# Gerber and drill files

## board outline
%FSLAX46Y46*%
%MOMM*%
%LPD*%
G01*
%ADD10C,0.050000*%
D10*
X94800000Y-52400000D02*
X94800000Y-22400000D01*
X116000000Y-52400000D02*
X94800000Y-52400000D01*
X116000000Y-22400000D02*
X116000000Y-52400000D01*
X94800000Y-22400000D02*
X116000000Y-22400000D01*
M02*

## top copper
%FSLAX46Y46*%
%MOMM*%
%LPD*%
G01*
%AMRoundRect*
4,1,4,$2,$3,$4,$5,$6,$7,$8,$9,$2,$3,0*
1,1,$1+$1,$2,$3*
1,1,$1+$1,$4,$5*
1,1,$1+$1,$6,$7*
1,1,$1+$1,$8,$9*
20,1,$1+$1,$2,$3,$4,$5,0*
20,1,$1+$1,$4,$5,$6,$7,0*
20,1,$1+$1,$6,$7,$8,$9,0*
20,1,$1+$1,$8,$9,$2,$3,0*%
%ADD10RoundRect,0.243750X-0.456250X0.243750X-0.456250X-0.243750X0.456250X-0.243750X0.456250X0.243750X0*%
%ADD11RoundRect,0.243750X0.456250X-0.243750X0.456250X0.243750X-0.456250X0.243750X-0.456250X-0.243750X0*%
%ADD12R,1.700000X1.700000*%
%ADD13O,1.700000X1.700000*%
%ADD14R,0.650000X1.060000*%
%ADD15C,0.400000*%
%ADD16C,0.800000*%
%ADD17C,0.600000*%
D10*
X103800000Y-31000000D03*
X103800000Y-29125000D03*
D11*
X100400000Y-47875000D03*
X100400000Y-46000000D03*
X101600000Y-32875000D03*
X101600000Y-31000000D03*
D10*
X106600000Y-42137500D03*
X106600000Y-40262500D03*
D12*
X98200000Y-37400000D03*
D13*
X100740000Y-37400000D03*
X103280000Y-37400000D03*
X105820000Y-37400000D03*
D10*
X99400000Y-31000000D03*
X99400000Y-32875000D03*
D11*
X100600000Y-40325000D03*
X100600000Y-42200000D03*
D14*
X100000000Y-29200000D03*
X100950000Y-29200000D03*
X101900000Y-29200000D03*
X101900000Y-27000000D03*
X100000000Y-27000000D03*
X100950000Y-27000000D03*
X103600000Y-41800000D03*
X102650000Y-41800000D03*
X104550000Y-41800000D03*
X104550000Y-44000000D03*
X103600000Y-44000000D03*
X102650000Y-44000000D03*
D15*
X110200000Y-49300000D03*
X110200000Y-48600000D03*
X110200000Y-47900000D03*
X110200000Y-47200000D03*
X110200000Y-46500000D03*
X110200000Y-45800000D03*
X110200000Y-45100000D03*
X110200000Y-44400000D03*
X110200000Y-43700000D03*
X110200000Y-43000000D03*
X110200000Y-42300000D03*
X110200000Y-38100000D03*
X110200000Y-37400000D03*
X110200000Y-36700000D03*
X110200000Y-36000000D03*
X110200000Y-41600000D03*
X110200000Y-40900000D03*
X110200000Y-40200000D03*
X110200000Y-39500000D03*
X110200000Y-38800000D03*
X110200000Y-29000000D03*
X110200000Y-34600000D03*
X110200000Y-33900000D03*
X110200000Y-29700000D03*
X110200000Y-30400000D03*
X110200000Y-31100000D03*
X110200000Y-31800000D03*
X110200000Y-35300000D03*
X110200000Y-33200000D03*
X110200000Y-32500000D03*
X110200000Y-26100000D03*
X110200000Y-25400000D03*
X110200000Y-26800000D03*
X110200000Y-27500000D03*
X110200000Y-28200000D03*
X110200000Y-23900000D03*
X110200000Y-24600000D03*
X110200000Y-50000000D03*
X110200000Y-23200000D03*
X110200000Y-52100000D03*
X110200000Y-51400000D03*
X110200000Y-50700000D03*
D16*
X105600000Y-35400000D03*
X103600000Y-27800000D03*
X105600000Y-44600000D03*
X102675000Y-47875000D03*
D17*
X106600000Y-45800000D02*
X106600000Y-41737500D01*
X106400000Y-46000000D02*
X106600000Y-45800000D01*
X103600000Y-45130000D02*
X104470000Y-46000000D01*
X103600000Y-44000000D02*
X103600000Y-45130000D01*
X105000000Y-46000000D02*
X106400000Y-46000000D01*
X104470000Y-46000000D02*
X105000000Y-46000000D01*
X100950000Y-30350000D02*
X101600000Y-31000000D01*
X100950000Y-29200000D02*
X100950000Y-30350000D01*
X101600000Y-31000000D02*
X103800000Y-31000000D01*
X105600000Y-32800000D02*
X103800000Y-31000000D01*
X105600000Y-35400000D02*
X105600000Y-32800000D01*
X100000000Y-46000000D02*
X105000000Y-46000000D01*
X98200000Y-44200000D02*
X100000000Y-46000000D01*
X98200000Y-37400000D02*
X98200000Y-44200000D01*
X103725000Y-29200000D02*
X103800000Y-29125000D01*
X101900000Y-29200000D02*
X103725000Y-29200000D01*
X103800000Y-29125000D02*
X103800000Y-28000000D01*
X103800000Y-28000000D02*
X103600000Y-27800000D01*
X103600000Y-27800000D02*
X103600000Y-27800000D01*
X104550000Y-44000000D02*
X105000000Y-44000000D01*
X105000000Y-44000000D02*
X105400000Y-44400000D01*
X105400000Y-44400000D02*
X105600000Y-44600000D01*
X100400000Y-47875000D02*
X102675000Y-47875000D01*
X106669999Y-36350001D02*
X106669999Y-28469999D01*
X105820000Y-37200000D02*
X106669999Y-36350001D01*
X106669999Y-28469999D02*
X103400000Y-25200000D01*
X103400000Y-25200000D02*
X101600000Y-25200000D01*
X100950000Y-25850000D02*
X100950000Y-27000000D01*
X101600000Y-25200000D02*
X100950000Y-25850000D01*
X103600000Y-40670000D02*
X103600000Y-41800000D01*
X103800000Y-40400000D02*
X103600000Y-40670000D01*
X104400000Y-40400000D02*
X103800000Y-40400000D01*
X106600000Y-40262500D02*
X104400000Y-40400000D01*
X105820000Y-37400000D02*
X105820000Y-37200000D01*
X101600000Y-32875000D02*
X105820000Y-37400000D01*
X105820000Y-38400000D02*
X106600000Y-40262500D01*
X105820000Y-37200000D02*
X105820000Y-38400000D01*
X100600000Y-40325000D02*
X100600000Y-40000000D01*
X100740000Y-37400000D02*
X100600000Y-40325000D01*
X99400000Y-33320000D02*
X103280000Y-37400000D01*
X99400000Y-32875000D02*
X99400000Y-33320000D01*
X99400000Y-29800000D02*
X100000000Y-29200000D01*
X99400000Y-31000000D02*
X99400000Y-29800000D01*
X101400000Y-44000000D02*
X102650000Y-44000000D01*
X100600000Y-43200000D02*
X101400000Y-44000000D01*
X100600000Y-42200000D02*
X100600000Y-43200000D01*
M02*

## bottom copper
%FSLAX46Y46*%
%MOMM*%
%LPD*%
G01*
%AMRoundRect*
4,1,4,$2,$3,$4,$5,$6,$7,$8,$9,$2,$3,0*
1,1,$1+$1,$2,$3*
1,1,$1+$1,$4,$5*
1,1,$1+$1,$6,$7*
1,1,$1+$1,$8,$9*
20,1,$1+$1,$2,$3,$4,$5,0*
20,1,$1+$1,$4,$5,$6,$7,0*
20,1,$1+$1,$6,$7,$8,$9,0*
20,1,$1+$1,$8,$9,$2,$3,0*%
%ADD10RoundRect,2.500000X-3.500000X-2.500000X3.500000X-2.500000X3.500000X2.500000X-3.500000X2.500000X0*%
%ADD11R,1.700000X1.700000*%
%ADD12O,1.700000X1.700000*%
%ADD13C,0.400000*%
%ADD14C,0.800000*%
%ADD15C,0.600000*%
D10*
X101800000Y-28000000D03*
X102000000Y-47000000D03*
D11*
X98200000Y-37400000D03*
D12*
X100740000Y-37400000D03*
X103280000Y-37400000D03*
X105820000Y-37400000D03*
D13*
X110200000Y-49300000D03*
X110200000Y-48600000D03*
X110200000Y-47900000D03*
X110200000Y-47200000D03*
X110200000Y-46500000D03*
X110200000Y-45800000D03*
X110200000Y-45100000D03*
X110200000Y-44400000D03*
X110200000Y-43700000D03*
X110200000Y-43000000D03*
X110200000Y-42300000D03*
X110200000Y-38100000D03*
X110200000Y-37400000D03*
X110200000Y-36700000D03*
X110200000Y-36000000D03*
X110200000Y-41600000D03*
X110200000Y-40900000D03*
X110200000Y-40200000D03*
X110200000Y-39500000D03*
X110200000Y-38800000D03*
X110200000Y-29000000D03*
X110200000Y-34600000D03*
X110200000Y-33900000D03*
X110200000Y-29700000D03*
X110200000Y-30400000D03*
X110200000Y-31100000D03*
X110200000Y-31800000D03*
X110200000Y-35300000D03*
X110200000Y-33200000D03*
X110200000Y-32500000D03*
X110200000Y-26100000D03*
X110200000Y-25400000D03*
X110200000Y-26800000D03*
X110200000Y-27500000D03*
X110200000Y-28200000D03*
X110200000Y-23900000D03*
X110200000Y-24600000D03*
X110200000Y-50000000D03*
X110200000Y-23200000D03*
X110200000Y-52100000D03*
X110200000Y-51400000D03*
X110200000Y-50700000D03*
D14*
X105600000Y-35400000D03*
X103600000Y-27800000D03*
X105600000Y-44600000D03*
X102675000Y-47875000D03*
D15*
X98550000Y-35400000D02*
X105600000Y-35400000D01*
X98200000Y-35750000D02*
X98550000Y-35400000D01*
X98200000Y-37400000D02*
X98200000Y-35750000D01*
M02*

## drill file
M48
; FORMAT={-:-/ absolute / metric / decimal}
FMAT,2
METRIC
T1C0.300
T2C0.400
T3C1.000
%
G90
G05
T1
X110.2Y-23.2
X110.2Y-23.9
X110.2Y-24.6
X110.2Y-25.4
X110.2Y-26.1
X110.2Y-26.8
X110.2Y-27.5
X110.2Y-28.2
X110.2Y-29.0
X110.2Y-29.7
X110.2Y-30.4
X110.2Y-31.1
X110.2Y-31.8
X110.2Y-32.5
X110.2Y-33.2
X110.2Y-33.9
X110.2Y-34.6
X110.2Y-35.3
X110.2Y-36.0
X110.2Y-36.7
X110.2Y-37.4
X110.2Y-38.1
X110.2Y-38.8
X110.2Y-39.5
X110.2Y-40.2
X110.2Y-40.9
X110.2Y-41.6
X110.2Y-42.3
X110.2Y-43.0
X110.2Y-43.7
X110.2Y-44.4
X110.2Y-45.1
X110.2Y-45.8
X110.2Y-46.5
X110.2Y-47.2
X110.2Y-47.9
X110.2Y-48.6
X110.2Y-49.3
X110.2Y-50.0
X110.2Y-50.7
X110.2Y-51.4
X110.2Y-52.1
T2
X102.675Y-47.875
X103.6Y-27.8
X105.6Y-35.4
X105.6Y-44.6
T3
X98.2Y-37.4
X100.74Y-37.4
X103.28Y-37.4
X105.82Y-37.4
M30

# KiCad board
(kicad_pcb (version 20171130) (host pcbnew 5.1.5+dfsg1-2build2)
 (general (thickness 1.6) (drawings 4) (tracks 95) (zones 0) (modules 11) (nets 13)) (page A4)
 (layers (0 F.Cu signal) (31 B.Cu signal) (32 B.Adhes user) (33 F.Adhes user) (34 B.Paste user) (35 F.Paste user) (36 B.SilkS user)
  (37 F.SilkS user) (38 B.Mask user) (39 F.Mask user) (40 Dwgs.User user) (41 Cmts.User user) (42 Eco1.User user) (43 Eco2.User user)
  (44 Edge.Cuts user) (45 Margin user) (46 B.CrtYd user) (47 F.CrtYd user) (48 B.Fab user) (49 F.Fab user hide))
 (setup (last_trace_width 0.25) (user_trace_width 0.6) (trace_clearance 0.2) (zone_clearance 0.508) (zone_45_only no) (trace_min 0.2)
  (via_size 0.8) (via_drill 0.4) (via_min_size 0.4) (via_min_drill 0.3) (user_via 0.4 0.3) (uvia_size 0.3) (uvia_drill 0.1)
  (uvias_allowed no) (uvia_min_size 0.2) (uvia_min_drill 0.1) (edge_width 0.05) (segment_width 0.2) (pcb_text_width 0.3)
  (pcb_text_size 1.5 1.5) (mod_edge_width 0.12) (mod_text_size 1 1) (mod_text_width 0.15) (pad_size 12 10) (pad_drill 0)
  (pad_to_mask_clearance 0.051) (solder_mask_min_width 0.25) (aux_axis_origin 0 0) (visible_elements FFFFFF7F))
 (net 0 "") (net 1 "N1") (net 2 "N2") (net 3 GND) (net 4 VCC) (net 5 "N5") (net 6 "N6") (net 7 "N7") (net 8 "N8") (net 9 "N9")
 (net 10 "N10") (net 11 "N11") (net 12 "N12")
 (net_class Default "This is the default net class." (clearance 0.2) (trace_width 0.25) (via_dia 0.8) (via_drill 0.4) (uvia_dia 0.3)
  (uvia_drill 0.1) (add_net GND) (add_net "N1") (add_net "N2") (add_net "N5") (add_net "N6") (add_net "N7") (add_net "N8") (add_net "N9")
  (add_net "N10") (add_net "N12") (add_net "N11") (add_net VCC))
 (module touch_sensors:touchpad (layer B.Cu) (at 101.8 28)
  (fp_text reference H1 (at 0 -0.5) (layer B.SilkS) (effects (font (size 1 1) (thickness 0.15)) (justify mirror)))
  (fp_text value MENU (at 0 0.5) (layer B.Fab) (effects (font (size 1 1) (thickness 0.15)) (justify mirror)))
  (pad 1 smd roundrect (at 0 0) (size 12 10) (layers B.Cu) (roundrect_rratio 0.25) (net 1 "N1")))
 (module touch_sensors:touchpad (layer B.Cu) (at 101.85 47)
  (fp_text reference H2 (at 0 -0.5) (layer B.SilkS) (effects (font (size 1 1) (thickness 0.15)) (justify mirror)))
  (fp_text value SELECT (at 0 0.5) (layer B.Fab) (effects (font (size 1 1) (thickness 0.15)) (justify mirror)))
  (pad 1 smd roundrect (at 0.15 0) (size 12 10) (layers B.Cu) (roundrect_rratio 0.25) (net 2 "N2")))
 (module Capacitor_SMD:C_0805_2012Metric (layer F.Cu) (at 103.8 30.0625 270)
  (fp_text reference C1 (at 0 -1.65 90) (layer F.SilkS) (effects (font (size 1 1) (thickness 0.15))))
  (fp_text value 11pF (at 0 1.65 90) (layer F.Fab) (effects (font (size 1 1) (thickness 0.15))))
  (pad 2 smd roundrect (at 0.9375 0 270) (size 0.975 1.4) (layers F.Cu F.Paste F.Mask) (roundrect_rratio 0.25) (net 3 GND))
  (pad 1 smd roundrect (at -0.9375 0 270) (size 0.975 1.4) (layers F.Cu F.Paste F.Mask) (roundrect_rratio 0.25) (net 1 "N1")))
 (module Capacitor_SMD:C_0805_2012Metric (layer F.Cu) (at 100.4 46.9375 90)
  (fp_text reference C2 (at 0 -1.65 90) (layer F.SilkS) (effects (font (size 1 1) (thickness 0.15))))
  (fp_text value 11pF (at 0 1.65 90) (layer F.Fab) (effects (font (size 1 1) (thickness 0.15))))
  (pad 1 smd roundrect (at -0.9375 0 90) (size 0.975 1.4) (layers F.Cu F.Paste F.Mask) (roundrect_rratio 0.25) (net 2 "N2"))
  (pad 2 smd roundrect (at 0.9375 0 90) (size 0.975 1.4) (layers F.Cu F.Paste F.Mask) (roundrect_rratio 0.25) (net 3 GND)))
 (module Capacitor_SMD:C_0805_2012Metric (layer F.Cu) (at 101.6 31.9375 90)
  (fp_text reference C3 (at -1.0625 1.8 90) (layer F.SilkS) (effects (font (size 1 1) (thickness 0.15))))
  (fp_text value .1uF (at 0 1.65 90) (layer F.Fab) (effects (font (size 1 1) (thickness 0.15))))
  (pad 1 smd roundrect (at -0.9375 0 90) (size 0.975 1.4) (layers F.Cu F.Paste F.Mask) (roundrect_rratio 0.25) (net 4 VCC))
  (pad 2 smd roundrect (at 0.9375 0 90) (size 0.975 1.4) (layers F.Cu F.Paste F.Mask) (roundrect_rratio 0.25) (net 3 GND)))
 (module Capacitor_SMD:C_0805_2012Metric (layer F.Cu) (at 106.6 41.2 270)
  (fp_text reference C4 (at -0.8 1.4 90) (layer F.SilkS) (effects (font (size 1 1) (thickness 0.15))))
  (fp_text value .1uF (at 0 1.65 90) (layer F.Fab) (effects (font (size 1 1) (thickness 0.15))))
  (pad 2 smd roundrect (at 0.9375 0 270) (size 0.975 1.4) (layers F.Cu F.Paste F.Mask) (roundrect_rratio 0.25) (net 3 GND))
  (pad 1 smd roundrect (at -0.9375 0 270) (size 0.975 1.4) (layers F.Cu F.Paste F.Mask) (roundrect_rratio 0.25) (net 4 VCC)))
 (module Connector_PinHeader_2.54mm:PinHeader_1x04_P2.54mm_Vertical (layer F.Cu) (at 98.2 37.4 90)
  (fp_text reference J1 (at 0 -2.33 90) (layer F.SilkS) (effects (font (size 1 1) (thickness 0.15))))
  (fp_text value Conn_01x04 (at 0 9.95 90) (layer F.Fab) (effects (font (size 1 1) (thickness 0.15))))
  (pad 1 thru_hole rect (at 0 0 90) (size 1.7 1.7) (drill 1) (layers *.Cu *.Mask) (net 3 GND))
  (pad 2 thru_hole oval (at 0 2.54 90) (size 1.7 1.7) (drill 1) (layers *.Cu *.Mask) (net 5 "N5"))
  (pad 3 thru_hole oval (at 0 5.08 90) (size 1.7 1.7) (drill 1) (layers *.Cu *.Mask) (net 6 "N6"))
  (pad 4 thru_hole oval (at 0 7.62 90) (size 1.7 1.7) (drill 1) (layers *.Cu *.Mask) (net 4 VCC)))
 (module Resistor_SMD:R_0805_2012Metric (layer F.Cu) (at 99.4 31.9375 270)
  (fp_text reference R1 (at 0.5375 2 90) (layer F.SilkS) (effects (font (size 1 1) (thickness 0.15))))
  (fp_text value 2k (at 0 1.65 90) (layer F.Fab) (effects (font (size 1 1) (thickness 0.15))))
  (pad 1 smd roundrect (at -0.9375 0 270) (size 0.975 1.4) (layers F.Cu F.Paste F.Mask) (roundrect_rratio 0.25) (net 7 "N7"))
  (pad 2 smd roundrect (at 0.9375 0 270) (size 0.975 1.4) (layers F.Cu F.Paste F.Mask) (roundrect_rratio 0.25) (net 6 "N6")))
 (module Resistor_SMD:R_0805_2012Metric (layer F.Cu) (at 100.6 41.2625 90)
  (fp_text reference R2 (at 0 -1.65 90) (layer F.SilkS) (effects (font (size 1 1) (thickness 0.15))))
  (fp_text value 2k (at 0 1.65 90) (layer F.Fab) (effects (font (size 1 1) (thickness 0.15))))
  (pad 2 smd roundrect (at 0.9375 0 90) (size 0.975 1.4) (layers F.Cu F.Paste F.Mask) (roundrect_rratio 0.25) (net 5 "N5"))
  (pad 1 smd roundrect (at -0.9375 0 90) (size 0.975 1.4) (layers F.Cu F.Paste F.Mask) (roundrect_rratio 0.25) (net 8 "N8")))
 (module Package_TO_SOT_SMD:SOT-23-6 (layer F.Cu) (at 100.95 28.1 90)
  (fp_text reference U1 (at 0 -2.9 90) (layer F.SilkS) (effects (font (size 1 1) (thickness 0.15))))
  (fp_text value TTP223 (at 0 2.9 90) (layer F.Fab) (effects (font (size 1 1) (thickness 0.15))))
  (pad 1 smd rect (at -1.1 -0.95 90) (size 1.06 0.65) (layers F.Cu F.Paste F.Mask) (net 7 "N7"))
  (pad 2 smd rect (at -1.1 0 90) (size 1.06 0.65) (layers F.Cu F.Paste F.Mask) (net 3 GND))
  (pad 3 smd rect (at -1.1 0.95 90) (size 1.06 0.65) (layers F.Cu F.Paste F.Mask) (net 1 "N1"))
  (pad 4 smd rect (at 1.1 0.95 90) (size 1.06 0.65) (layers F.Cu F.Paste F.Mask) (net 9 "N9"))
  (pad 6 smd rect (at 1.1 -0.95 90) (size 1.06 0.65) (layers F.Cu F.Paste F.Mask) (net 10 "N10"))
  (pad 5 smd rect (at 1.1 0 90) (size 1.06 0.65) (layers F.Cu F.Paste F.Mask) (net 4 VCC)))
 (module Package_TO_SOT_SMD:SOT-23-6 (layer F.Cu) (at 103.6 42.9 90)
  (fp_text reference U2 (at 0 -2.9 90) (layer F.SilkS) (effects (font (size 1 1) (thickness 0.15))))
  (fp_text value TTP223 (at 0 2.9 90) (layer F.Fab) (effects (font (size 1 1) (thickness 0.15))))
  (pad 5 smd rect (at 1.1 0 90) (size 1.06 0.65) (layers F.Cu F.Paste F.Mask) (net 4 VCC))
  (pad 6 smd rect (at 1.1 -0.95 90) (size 1.06 0.65) (layers F.Cu F.Paste F.Mask) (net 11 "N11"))
  (pad 4 smd rect (at 1.1 0.95 90) (size 1.06 0.65) (layers F.Cu F.Paste F.Mask) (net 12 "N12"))
  (pad 3 smd rect (at -1.1 0.95 90) (size 1.06 0.65) (layers F.Cu F.Paste F.Mask) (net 2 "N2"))
  (pad 2 smd rect (at -1.1 0 90) (size 1.06 0.65) (layers F.Cu F.Paste F.Mask) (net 3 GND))
  (pad 1 smd rect (at -1.1 -0.95 90) (size 1.06 0.65) (layers F.Cu F.Paste F.Mask) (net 8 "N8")))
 (gr_line (start 94.8 52.4) (end 94.8 22.4) (layer Edge.Cuts) (width 0.05))
 (gr_line (start 116 52.4) (end 94.8 52.4) (layer Edge.Cuts) (width 0.05))
 (gr_line (start 116 22.4) (end 116 52.4) (layer Edge.Cuts) (width 0.05))
 (gr_line (start 94.8 22.4) (end 116 22.4) (layer Edge.Cuts) (width 0.05))
 (via (at 110.2 49.3) (size 0.4) (drill 0.3) (layers F.Cu B.Cu) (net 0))
 (via (at 110.2 48.6) (size 0.4) (drill 0.3) (layers F.Cu B.Cu) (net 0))
 (via (at 110.2 47.9) (size 0.4) (drill 0.3) (layers F.Cu B.Cu) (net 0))
 (via (at 110.2 47.2) (size 0.4) (drill 0.3) (layers F.Cu B.Cu) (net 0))
 (via (at 110.2 46.5) (size 0.4) (drill 0.3) (layers F.Cu B.Cu) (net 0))
 (via (at 110.2 45.8) (size 0.4) (drill 0.3) (layers F.Cu B.Cu) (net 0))
 (via (at 110.2 45.1) (size 0.4) (drill 0.3) (layers F.Cu B.Cu) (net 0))
 (via (at 110.2 44.4) (size 0.4) (drill 0.3) (layers F.Cu B.Cu) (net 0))
 (via (at 110.2 43.7) (size 0.4) (drill 0.3) (layers F.Cu B.Cu) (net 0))
 (via (at 110.2 43) (size 0.4) (drill 0.3) (layers F.Cu B.Cu) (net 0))
 (via (at 110.2 42.3) (size 0.4) (drill 0.3) (layers F.Cu B.Cu) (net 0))
 (via (at 110.2 38.1) (size 0.4) (drill 0.3) (layers F.Cu B.Cu) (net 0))
 (via (at 110.2 37.4) (size 0.4) (drill 0.3) (layers F.Cu B.Cu) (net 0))
 (via (at 110.2 36.7) (size 0.4) (drill 0.3) (layers F.Cu B.Cu) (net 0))
 (via (at 110.2 36) (size 0.4) (drill 0.3) (layers F.Cu B.Cu) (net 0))
 (via (at 110.2 41.6) (size 0.4) (drill 0.3) (layers F.Cu B.Cu) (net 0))
 (via (at 110.2 40.9) (size 0.4) (drill 0.3) (layers F.Cu B.Cu) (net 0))
 (via (at 110.2 40.2) (size 0.4) (drill 0.3) (layers F.Cu B.Cu) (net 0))
 (via (at 110.2 39.5) (size 0.4) (drill 0.3) (layers F.Cu B.Cu) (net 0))
 (via (at 110.2 38.8) (size 0.4) (drill 0.3) (layers F.Cu B.Cu) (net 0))
 (via (at 110.2 29) (size 0.4) (drill 0.3) (layers F.Cu B.Cu) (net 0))
 (via (at 110.2 34.6) (size 0.4) (drill 0.3) (layers F.Cu B.Cu) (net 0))
 (via (at 110.2 33.9) (size 0.4) (drill 0.3) (layers F.Cu B.Cu) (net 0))
 (via (at 110.2 29.7) (size 0.4) (drill 0.3) (layers F.Cu B.Cu) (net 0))
 (via (at 110.2 30.4) (size 0.4) (drill 0.3) (layers F.Cu B.Cu) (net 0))
 (via (at 110.2 31.1) (size 0.4) (drill 0.3) (layers F.Cu B.Cu) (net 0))
 (via (at 110.2 31.8) (size 0.4) (drill 0.3) (layers F.Cu B.Cu) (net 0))
 (via (at 110.2 35.3) (size 0.4) (drill 0.3) (layers F.Cu B.Cu) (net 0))
 (via (at 110.2 33.2) (size 0.4) (drill 0.3) (layers F.Cu B.Cu) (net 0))
 (via (at 110.2 32.5) (size 0.4) (drill 0.3) (layers F.Cu B.Cu) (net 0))
 (via (at 110.2 26.1) (size 0.4) (drill 0.3) (layers F.Cu B.Cu) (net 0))
 (via (at 110.2 25.4) (size 0.4) (drill 0.3) (layers F.Cu B.Cu) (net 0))
 (via (at 110.2 26.8) (size 0.4) (drill 0.3) (layers F.Cu B.Cu) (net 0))
 (via (at 110.2 27.5) (size 0.4) (drill 0.3) (layers F.Cu B.Cu) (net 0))
 (via (at 110.2 28.2) (size 0.4) (drill 0.3) (layers F.Cu B.Cu) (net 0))
 (via (at 110.2 23.9) (size 0.4) (drill 0.3) (layers F.Cu B.Cu) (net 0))
 (via (at 110.2 24.6) (size 0.4) (drill 0.3) (layers F.Cu B.Cu) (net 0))
 (via (at 110.2 50) (size 0.4) (drill 0.3) (layers F.Cu B.Cu) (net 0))
 (via (at 110.2 23.2) (size 0.4) (drill 0.3) (layers F.Cu B.Cu) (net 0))
 (via (at 110.2 52.1) (size 0.4) (drill 0.3) (layers F.Cu B.Cu) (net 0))
 (via (at 110.2 51.4) (size 0.4) (drill 0.3) (layers F.Cu B.Cu) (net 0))
 (via (at 110.2 50.7) (size 0.4) (drill 0.3) (layers F.Cu B.Cu) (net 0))
 (segment (start 106.6 45.8) (end 106.6 41.7375) (width 0.6) (layer F.Cu) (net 3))
 (segment (start 106.4 46) (end 106.6 45.8) (width 0.6) (layer F.Cu) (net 3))
 (segment (start 103.6 45.13) (end 104.47 46) (width 0.6) (layer F.Cu) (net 3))
 (segment (start 103.6 44) (end 103.6 45.13) (width 0.6) (layer F.Cu) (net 3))
 (segment (start 105 46) (end 106.4 46) (width 0.6) (layer F.Cu) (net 3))
 (segment (start 104.47 46) (end 105 46) (width 0.6) (layer F.Cu) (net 3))
 (segment (start 100.95 30.35) (end 101.6 31) (width 0.6) (layer F.Cu) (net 3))
 (segment (start 100.95 29.2) (end 100.95 30.35) (width 0.6) (layer F.Cu) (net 3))
 (segment (start 101.6 31) (end 103.8 31) (width 0.6) (layer F.Cu) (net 3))
 (via (at 105.6 35.4) (size 0.8) (drill 0.4) (layers F.Cu B.Cu) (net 3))
 (segment (start 105.6 32.8) (end 103.8 31) (width 0.6) (layer F.Cu) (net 3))
 (segment (start 105.6 35.4) (end 105.6 32.8) (width 0.6) (layer F.Cu) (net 3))
 (segment (start 100 46) (end 105 46) (width 0.6) (layer F.Cu) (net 3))
 (segment (start 98.2 44.2) (end 100 46) (width 0.6) (layer F.Cu) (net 3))
 (segment (start 98.2 37.4) (end 98.2 44.2) (width 0.6) (layer F.Cu) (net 3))
 (segment (start 98.55 35.4) (end 105.6 35.4) (width 0.6) (layer B.Cu) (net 3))
 (segment (start 98.2 35.75) (end 98.55 35.4) (width 0.6) (layer B.Cu) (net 3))
 (segment (start 98.2 37.4) (end 98.2 35.75) (width 0.6) (layer B.Cu) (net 3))
 (segment (start 103.725 29.2) (end 103.8 29.125) (width 0.6) (layer F.Cu) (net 1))
 (segment (start 101.9 29.2) (end 103.725 29.2) (width 0.6) (layer F.Cu) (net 1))
 (segment (start 103.8 29.125) (end 103.8 28) (width 0.6) (layer F.Cu) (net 1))
 (segment (start 103.8 28) (end 103.6 27.8) (width 0.6) (layer F.Cu) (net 1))
 (segment (start 103.6 27.8) (end 103.6 27.8) (width 0.6) (layer F.Cu) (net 1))
 (via (at 103.6 27.8) (size 0.8) (drill 0.4) (layers F.Cu B.Cu) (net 1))
 (segment (start 104.55 44) (end 105 44) (width 0.6) (layer F.Cu) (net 2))
 (segment (start 105 44) (end 105.4 44.4) (width 0.6) (layer F.Cu) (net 2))
 (segment (start 105.4 44.4) (end 105.6 44.6) (width 0.6) (layer F.Cu) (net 2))
 (via (at 105.6 44.6) (size 0.8) (drill 0.4) (layers F.Cu B.Cu) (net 2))
 (segment (start 100.4 47.875) (end 102.675 47.875) (width 0.6) (layer F.Cu) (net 2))
 (via (at 102.675 47.875) (size 0.8) (drill 0.4) (layers F.Cu B.Cu) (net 2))
 (segment (start 106.669999 36.350001) (end 106.669999 28.469999) (width 0.6) (layer F.Cu) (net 4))
 (segment (start 105.82 37.2) (end 106.669999 36.350001) (width 0.6) (layer F.Cu) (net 4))
 (segment (start 106.669999 28.469999) (end 103.4 25.2) (width 0.6) (layer F.Cu) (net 4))
 (segment (start 103.4 25.2) (end 101.6 25.2) (width 0.6) (layer F.Cu) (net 4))
 (segment (start 100.95 25.85) (end 100.95 27) (width 0.6) (layer F.Cu) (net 4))
 (segment (start 101.6 25.2) (end 100.95 25.85) (width 0.6) (layer F.Cu) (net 4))
 (segment (start 103.6 40.67) (end 103.6 41.8) (width 0.6) (layer F.Cu) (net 4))
 (segment (start 103.8 40.4) (end 103.6 40.67) (width 0.6) (layer F.Cu) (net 4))
 (segment (start 104.4 40.4) (end 103.8 40.4) (width 0.6) (layer F.Cu) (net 4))
 (segment (start 106.6 40.2625) (end 104.4 40.4) (width 0.6) (layer F.Cu) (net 4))
 (segment (start 105.82 37.4) (end 105.82 37.2) (width 0.6) (layer F.Cu) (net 4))
 (segment (start 101.6 32.875) (end 105.82 37.4) (width 0.6) (layer F.Cu) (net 4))
 (segment (start 105.82 38.4) (end 106.6 40.2625) (width 0.6) (layer F.Cu) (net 4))
 (segment (start 105.82 37.2) (end 105.82 38.4) (width 0.6) (layer F.Cu) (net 4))
 (segment (start 100.6 40.325) (end 100.6 40) (width 0.6) (layer F.Cu) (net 5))
 (segment (start 100.74 37.4) (end 100.6 40.325) (width 0.6) (layer F.Cu) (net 5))
 (segment (start 99.4 33.32) (end 103.28 37.4) (width 0.6) (layer F.Cu) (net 6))
 (segment (start 99.4 32.875) (end 99.4 33.32) (width 0.6) (layer F.Cu) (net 6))
 (segment (start 99.4 29.8) (end 100 29.2) (width 0.6) (layer F.Cu) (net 7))
 (segment (start 99.4 31) (end 99.4 29.8) (width 0.6) (layer F.Cu) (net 7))
 (segment (start 101.4 44) (end 102.65 44) (width 0.6) (layer F.Cu) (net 8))
 (segment (start 100.6 43.2) (end 101.4 44) (width 0.6) (layer F.Cu) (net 8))
 (segment (start 100.6 42.2) (end 100.6 43.2) (width 0.6) (layer F.Cu) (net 8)))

